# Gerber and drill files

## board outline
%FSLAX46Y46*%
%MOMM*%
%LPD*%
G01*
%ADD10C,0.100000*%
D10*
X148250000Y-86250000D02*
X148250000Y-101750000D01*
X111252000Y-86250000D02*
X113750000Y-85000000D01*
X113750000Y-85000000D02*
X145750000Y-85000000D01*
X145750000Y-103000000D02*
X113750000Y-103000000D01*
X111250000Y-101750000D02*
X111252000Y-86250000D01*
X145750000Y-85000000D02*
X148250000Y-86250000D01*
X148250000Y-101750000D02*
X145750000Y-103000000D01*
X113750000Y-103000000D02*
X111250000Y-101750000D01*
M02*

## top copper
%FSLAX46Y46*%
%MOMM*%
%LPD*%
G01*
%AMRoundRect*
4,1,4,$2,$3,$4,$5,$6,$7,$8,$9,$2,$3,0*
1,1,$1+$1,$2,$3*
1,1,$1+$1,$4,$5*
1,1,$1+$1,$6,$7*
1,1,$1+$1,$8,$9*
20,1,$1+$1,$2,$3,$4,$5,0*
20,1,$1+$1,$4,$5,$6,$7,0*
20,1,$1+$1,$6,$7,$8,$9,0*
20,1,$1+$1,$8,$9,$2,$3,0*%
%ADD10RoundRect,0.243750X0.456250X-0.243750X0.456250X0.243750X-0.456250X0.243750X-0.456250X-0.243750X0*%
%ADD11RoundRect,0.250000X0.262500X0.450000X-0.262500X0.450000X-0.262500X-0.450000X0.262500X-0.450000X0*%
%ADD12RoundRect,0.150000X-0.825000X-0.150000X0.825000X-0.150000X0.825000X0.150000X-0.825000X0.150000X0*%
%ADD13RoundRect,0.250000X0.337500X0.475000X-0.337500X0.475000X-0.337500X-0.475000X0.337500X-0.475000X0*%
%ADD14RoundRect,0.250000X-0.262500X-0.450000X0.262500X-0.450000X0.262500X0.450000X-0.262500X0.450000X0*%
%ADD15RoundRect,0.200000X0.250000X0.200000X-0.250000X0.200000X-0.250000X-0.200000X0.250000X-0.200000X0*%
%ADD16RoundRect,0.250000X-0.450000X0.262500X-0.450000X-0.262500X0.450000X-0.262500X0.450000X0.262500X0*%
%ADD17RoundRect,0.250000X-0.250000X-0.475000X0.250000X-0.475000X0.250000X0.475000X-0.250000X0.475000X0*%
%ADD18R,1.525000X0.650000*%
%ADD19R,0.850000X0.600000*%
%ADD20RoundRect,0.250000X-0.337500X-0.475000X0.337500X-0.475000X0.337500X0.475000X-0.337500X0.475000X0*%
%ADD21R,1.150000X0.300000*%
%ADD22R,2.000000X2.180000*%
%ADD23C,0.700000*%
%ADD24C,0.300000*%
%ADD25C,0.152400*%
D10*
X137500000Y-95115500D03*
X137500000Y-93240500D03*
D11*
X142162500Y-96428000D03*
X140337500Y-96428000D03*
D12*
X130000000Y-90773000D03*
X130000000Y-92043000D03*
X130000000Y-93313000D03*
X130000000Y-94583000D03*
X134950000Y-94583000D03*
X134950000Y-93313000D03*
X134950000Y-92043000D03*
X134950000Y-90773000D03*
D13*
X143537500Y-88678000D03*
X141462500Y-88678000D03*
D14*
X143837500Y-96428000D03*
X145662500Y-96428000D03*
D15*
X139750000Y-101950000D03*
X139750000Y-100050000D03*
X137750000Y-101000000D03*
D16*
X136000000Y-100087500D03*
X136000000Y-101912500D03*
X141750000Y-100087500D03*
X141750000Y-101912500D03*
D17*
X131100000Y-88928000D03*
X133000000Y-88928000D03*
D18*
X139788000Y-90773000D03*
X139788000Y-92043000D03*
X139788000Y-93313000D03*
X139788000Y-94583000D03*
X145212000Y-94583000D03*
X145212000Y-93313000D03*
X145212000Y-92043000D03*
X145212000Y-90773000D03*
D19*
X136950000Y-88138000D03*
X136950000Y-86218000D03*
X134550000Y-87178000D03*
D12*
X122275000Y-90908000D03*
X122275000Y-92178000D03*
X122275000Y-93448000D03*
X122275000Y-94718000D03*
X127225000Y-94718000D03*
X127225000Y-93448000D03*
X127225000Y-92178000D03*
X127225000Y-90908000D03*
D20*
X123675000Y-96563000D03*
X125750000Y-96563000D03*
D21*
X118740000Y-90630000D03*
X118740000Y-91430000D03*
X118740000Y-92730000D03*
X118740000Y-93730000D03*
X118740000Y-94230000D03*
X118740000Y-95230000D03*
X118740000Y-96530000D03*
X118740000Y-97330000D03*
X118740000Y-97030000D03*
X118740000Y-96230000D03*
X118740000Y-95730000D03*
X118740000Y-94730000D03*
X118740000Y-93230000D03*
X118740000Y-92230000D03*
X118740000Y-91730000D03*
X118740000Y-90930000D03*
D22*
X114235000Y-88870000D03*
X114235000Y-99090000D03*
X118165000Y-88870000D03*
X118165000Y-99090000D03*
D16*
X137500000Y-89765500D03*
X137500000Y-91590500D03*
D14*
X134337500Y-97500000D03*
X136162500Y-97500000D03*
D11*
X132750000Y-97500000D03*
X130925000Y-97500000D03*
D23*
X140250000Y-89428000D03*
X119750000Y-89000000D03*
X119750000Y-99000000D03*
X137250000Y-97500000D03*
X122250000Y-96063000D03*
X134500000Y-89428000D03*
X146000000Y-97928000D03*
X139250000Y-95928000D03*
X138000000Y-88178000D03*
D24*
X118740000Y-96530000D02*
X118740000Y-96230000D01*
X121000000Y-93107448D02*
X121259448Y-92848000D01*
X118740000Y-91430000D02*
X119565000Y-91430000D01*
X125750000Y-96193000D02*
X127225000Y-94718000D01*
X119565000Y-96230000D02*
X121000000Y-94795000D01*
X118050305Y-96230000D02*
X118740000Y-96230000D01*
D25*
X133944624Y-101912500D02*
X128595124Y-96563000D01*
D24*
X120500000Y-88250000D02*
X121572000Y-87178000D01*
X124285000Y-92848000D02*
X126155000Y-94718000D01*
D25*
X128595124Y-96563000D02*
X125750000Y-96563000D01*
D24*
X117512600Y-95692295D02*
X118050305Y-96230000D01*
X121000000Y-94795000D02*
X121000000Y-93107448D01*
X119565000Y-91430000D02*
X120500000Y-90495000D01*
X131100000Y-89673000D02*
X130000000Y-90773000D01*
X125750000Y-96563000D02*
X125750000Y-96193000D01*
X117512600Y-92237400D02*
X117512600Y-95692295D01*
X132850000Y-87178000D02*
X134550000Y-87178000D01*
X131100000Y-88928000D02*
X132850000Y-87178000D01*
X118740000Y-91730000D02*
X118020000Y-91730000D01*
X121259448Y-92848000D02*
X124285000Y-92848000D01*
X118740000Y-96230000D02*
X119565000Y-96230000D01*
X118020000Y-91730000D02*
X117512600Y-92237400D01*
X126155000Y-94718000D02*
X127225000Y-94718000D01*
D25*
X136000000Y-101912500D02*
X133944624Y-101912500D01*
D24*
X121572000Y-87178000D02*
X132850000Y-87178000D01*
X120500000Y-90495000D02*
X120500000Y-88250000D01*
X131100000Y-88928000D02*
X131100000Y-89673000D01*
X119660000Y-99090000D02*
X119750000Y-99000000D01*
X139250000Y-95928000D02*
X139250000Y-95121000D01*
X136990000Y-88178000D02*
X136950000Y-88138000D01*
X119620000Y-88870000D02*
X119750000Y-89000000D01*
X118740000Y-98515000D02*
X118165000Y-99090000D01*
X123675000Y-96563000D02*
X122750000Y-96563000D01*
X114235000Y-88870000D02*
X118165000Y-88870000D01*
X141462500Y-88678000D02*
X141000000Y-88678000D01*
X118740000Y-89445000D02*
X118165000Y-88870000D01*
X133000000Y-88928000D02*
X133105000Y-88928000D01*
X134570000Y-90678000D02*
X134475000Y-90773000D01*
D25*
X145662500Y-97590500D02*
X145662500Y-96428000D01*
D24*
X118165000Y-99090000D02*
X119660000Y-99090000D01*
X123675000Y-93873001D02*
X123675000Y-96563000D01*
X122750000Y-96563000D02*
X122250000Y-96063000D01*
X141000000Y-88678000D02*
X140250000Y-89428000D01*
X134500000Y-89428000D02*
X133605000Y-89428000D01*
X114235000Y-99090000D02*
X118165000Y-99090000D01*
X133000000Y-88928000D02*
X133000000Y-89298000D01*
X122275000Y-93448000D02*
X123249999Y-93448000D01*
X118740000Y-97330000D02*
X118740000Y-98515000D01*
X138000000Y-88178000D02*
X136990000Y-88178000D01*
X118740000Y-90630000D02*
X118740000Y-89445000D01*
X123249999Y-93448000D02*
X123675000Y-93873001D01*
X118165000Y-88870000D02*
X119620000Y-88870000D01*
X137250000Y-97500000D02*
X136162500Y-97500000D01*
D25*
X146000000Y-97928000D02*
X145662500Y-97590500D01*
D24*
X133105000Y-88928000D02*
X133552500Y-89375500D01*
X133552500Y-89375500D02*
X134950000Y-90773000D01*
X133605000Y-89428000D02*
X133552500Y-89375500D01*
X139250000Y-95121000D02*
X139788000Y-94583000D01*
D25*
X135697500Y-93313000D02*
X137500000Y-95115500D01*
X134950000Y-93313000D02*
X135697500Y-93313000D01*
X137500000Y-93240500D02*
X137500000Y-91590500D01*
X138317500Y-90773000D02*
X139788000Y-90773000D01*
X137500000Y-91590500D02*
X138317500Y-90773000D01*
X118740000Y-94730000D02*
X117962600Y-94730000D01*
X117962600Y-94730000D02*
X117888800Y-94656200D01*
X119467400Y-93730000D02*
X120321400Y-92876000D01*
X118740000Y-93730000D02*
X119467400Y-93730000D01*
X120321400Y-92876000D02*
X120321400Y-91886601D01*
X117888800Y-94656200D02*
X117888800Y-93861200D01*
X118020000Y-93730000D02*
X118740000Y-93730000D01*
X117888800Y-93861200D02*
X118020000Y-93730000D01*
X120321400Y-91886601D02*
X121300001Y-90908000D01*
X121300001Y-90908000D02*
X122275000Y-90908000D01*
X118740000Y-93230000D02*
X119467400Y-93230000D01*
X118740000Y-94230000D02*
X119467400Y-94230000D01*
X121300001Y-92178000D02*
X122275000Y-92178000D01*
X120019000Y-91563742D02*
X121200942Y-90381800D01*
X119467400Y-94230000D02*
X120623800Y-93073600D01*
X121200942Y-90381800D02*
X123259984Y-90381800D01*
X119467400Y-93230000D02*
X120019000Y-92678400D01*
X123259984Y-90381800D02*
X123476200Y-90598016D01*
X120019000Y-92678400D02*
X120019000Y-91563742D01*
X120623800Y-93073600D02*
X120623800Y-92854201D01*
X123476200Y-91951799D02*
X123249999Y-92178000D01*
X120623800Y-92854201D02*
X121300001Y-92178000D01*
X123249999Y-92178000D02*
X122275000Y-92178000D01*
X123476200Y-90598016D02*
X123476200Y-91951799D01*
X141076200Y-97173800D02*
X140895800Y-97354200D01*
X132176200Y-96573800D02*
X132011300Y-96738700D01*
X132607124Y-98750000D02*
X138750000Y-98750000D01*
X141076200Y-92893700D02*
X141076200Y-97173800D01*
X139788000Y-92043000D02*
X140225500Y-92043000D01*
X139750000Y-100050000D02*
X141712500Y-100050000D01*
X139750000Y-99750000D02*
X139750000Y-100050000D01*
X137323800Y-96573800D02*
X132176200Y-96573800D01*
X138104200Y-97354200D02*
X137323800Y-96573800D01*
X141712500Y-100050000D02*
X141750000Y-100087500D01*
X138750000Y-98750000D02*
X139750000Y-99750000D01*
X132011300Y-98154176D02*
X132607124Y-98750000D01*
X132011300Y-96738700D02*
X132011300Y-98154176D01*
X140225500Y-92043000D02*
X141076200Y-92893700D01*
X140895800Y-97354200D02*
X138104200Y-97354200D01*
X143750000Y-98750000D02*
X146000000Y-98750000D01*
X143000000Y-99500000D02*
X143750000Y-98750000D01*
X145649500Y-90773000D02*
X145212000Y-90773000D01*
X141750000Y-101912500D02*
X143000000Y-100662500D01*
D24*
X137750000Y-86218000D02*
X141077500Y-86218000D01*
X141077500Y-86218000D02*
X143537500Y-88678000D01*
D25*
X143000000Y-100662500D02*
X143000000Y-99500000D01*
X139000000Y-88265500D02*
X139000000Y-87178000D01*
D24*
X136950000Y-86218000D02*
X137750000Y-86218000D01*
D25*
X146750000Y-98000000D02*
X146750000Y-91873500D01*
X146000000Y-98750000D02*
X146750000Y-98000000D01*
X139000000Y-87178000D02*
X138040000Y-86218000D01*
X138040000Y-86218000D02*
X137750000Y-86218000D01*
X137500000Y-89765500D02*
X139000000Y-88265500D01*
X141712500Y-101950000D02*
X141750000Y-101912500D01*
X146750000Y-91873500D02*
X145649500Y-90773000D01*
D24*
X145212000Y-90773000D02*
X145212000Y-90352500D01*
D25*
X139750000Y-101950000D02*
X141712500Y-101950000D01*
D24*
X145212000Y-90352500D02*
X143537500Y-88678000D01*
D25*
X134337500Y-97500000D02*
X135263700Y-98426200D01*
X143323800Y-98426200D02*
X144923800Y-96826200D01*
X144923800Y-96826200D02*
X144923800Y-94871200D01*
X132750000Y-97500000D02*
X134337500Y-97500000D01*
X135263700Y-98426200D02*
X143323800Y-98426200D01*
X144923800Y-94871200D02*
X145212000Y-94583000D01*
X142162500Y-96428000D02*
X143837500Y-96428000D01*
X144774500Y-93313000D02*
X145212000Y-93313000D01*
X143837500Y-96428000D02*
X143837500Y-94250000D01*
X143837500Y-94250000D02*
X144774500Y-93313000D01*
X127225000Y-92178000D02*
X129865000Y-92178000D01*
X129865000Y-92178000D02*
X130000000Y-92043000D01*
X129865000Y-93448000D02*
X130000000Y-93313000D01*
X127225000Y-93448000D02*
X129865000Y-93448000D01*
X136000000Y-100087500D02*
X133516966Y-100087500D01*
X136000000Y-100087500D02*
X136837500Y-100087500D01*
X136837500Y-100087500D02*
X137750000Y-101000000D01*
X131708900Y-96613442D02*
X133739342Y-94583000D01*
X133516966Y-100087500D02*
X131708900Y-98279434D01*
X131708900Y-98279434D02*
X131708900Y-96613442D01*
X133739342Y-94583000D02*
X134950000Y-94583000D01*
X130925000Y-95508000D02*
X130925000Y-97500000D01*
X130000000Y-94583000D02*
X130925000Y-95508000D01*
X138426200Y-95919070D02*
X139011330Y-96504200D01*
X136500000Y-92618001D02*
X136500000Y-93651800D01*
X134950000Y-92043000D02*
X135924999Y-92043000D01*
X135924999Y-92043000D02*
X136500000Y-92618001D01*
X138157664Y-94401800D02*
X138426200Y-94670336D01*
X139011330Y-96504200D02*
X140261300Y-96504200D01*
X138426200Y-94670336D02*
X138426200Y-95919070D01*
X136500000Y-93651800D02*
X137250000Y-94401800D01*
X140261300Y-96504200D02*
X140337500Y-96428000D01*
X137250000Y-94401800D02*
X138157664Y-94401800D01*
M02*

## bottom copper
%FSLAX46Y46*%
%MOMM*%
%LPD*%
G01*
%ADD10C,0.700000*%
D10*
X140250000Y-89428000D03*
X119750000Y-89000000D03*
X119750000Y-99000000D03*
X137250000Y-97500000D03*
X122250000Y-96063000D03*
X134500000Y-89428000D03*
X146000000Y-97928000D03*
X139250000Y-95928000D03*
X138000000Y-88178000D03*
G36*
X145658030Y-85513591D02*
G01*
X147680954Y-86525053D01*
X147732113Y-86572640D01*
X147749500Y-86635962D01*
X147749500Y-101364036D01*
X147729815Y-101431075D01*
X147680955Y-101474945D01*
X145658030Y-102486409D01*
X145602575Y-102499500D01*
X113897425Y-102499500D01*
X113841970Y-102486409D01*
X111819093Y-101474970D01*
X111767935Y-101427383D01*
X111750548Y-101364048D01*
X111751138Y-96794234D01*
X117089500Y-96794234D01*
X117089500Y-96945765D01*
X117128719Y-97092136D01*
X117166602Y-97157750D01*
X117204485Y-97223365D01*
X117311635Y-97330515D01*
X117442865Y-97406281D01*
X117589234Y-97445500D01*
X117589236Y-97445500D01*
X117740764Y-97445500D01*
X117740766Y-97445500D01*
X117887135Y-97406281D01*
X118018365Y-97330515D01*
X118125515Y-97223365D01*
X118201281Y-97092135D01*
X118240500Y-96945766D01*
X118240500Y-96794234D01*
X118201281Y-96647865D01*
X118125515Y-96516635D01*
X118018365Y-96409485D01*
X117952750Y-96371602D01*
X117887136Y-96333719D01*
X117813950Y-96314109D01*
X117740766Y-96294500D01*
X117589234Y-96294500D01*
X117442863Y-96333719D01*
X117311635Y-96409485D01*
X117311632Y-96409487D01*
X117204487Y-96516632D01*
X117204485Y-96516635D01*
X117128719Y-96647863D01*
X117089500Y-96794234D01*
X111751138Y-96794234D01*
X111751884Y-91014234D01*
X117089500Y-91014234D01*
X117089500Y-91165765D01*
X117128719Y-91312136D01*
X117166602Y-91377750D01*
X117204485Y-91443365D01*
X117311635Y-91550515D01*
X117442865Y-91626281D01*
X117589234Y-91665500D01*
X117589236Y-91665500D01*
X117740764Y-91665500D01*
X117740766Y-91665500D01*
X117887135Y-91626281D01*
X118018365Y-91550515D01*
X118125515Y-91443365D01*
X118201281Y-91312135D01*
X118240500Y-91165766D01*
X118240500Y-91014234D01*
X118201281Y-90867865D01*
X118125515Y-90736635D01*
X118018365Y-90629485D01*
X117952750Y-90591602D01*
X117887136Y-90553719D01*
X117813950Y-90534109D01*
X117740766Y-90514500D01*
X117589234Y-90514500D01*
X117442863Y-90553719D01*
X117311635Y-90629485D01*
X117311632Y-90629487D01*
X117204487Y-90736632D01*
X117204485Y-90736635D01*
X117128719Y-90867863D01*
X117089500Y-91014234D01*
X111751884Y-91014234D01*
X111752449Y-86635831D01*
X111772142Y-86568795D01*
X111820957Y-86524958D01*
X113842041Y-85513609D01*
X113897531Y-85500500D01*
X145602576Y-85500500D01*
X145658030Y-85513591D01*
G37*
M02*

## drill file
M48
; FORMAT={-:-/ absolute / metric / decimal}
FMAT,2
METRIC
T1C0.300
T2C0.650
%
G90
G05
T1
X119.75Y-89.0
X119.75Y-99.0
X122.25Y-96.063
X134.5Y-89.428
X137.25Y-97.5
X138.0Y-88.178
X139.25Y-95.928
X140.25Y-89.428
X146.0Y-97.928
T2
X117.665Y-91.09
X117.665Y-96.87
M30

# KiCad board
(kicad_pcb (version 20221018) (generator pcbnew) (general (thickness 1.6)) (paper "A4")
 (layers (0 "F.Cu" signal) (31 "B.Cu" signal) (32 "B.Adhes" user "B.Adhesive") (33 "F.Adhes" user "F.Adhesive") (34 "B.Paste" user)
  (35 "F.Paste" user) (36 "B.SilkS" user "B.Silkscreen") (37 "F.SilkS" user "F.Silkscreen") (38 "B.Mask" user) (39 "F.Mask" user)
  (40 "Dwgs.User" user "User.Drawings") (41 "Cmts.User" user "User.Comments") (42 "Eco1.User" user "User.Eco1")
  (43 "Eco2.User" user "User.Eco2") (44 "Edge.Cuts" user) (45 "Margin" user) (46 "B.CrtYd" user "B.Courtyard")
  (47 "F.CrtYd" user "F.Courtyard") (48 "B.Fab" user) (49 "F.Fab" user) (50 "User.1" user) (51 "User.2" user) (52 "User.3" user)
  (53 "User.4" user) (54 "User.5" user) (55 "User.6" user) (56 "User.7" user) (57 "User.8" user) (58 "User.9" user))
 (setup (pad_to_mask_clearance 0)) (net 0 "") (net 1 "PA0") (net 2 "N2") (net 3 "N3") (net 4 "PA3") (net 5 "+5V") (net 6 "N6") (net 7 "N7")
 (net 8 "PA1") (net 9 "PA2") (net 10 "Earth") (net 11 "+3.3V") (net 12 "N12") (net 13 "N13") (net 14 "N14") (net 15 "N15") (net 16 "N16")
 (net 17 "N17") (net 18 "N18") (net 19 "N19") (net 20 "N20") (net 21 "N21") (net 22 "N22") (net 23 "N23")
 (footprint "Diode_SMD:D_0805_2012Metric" (layer "F.Cu") (at 137.5 94.178 90)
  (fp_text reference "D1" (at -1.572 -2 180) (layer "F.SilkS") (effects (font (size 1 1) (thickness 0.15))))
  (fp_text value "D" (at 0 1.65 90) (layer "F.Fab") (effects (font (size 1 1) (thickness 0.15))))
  (pad "1" smd roundrect (at -0.9375 0 90) (size 0.975 1.4) (layers "F.Cu" "F.Paste" "F.Mask") (roundrect_rratio 0.25) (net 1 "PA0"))
  (pad "2" smd roundrect (at 0.9375 0 90) (size 0.975 1.4) (layers "F.Cu" "F.Paste" "F.Mask") (roundrect_rratio 0.25) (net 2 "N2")))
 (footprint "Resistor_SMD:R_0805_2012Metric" (layer "F.Cu") (at 141.25 96.428 180)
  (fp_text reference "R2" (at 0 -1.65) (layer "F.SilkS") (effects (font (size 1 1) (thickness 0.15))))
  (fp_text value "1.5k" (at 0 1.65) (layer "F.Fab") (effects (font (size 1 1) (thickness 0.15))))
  (pad "1" smd roundrect (at -0.9125 0 180) (size 1.025 1.4) (layers "F.Cu" "F.Paste" "F.Mask") (roundrect_rratio 0.243902) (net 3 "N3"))
  (pad "2" smd roundrect (at 0.9125 0 180) (size 1.025 1.4) (layers "F.Cu" "F.Paste" "F.Mask") (roundrect_rratio 0.243902) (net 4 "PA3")))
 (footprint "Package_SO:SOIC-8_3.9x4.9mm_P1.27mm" (layer "F.Cu") (at 132.475 92.678)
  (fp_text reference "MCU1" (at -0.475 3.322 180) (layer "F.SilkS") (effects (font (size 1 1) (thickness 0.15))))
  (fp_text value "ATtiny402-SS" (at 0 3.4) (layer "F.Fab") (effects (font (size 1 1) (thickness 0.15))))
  (pad "1" smd roundrect (at -2.475 -1.905) (size 1.95 0.6) (layers "F.Cu" "F.Paste" "F.Mask") (roundrect_rratio 0.25) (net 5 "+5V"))
  (pad "2" smd roundrect (at -2.475 -0.635) (size 1.95 0.6) (layers "F.Cu" "F.Paste" "F.Mask") (roundrect_rratio 0.25) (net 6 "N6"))
  (pad "3" smd roundrect (at -2.475 0.635) (size 1.95 0.6) (layers "F.Cu" "F.Paste" "F.Mask") (roundrect_rratio 0.25) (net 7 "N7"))
  (pad "4" smd roundrect (at -2.475 1.905) (size 1.95 0.6) (layers "F.Cu" "F.Paste" "F.Mask") (roundrect_rratio 0.25) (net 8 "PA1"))
  (pad "5" smd roundrect (at 2.475 1.905) (size 1.95 0.6) (layers "F.Cu" "F.Paste" "F.Mask") (roundrect_rratio 0.25) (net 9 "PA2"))
  (pad "6" smd roundrect (at 2.475 0.635) (size 1.95 0.6) (layers "F.Cu" "F.Paste" "F.Mask") (roundrect_rratio 0.25) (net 1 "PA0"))
  (pad "7" smd roundrect (at 2.475 -0.635) (size 1.95 0.6) (layers "F.Cu" "F.Paste" "F.Mask") (roundrect_rratio 0.25) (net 4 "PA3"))
  (pad "8" smd roundrect (at 2.475 -1.905) (size 1.95 0.6) (layers "F.Cu" "F.Paste" "F.Mask") (roundrect_rratio 0.25) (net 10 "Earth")))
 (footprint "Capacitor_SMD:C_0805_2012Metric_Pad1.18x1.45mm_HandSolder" (layer "F.Cu") (at 142.5 88.678 180)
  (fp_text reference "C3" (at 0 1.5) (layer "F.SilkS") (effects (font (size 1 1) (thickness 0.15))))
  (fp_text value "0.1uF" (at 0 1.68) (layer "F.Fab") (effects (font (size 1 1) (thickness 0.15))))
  (pad "1" smd roundrect (at -1.0375 0 180) (size 1.175 1.45) (layers "F.Cu" "F.Paste" "F.Mask") (roundrect_rratio 0.212766)
   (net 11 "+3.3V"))
  (pad "2" smd roundrect (at 1.0375 0 180) (size 1.175 1.45) (layers "F.Cu" "F.Paste" "F.Mask") (roundrect_rratio 0.212766) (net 10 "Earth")))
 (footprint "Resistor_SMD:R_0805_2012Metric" (layer "F.Cu") (at 144.75 96.428)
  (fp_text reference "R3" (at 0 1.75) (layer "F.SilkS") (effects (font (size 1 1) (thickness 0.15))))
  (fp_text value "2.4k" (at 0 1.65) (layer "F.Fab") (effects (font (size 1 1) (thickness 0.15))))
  (pad "1" smd roundrect (at -0.9125 0) (size 1.025 1.4) (layers "F.Cu" "F.Paste" "F.Mask") (roundrect_rratio 0.243902) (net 3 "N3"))
  (pad "2" smd roundrect (at 0.9125 0) (size 1.025 1.4) (layers "F.Cu" "F.Paste" "F.Mask") (roundrect_rratio 0.243902) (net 10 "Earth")))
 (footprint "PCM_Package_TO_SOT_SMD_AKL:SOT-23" (layer "F.Cu") (at 138.75 101 180)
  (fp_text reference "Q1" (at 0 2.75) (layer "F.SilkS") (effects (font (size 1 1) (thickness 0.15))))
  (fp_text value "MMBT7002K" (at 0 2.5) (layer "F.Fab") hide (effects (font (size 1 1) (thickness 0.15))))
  (pad "1" smd roundrect (at -1 -0.95 180) (size 0.9 0.8) (layers "F.Cu" "F.Paste" "F.Mask") (roundrect_rratio 0.25) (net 11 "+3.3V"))
  (pad "2" smd roundrect (at -1 0.95 180) (size 0.9 0.8) (layers "F.Cu" "F.Paste" "F.Mask") (roundrect_rratio 0.25) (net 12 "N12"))
  (pad "3" smd roundrect (at 1 0 180) (size 0.9 0.8) (layers "F.Cu" "F.Paste" "F.Mask") (roundrect_rratio 0.25) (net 9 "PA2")))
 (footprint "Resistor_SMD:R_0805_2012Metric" (layer "F.Cu") (at 136 101 -90)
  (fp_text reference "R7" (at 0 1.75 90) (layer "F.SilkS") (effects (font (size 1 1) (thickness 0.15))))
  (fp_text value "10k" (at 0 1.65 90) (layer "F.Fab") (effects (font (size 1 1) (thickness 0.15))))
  (pad "1" smd roundrect (at -0.9125 0 270) (size 1.025 1.4) (layers "F.Cu" "F.Paste" "F.Mask") (roundrect_rratio 0.243902) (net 9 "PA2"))
  (pad "2" smd roundrect (at 0.9125 0 270) (size 1.025 1.4) (layers "F.Cu" "F.Paste" "F.Mask") (roundrect_rratio 0.243902) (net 5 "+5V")))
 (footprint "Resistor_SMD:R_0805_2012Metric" (layer "F.Cu") (at 141.75 101 -90)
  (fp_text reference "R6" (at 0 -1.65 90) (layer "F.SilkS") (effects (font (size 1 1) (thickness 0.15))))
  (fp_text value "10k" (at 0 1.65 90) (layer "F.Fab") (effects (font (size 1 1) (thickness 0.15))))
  (pad "1" smd roundrect (at -0.9125 0 270) (size 1.025 1.4) (layers "F.Cu" "F.Paste" "F.Mask") (roundrect_rratio 0.243902) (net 12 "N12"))
  (pad "2" smd roundrect (at 0.9125 0 270) (size 1.025 1.4) (layers "F.Cu" "F.Paste" "F.Mask") (roundrect_rratio 0.243902) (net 11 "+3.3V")))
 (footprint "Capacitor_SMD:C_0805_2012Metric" (layer "F.Cu") (at 132.05 88.928)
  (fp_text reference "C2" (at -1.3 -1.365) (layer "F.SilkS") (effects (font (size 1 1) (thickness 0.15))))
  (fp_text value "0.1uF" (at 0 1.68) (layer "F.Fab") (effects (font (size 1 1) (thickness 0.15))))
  (pad "1" smd roundrect (at -0.95 0) (size 1 1.45) (layers "F.Cu" "F.Paste" "F.Mask") (roundrect_rratio 0.25) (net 5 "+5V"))
  (pad "2" smd roundrect (at 0.95 0) (size 1 1.45) (layers "F.Cu" "F.Paste" "F.Mask") (roundrect_rratio 0.25) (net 10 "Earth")))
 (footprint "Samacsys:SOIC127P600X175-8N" (layer "F.Cu") (at 142.5 92.678)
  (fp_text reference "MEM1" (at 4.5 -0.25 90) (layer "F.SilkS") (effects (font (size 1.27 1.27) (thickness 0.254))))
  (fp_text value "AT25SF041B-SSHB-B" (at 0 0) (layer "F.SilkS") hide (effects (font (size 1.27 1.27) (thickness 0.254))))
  (pad "1" smd rect (at -2.712 -1.905 90) (size 0.65 1.525) (layers "F.Cu" "F.Paste" "F.Mask") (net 2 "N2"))
  (pad "2" smd rect (at -2.712 -0.635 90) (size 0.65 1.525) (layers "F.Cu" "F.Paste" "F.Mask") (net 12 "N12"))
  (pad "3" smd rect (at -2.712 0.635 90) (size 0.65 1.525) (layers "F.Cu" "F.Paste" "F.Mask") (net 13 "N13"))
  (pad "4" smd rect (at -2.712 1.905 90) (size 0.65 1.525) (layers "F.Cu" "F.Paste" "F.Mask") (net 10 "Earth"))
  (pad "5" smd rect (at 2.712 1.905 90) (size 0.65 1.525) (layers "F.Cu" "F.Paste" "F.Mask") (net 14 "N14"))
  (pad "6" smd rect (at 2.712 0.635 90) (size 0.65 1.525) (layers "F.Cu" "F.Paste" "F.Mask") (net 3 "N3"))
  (pad "7" smd rect (at 2.712 -0.635 90) (size 0.65 1.525) (layers "F.Cu" "F.Paste" "F.Mask") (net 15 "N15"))
  (pad "8" smd rect (at 2.712 -1.905 90) (size 0.65 1.525) (layers "F.Cu" "F.Paste" "F.Mask") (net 11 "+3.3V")))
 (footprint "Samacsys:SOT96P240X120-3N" (layer "F.Cu") (at 135.75 87.178 180)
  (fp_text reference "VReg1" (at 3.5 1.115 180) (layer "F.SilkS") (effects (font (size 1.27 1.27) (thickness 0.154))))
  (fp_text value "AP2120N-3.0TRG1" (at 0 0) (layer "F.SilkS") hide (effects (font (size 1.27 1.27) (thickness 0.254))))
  (pad "1" smd rect (at -1.2 -0.96 270) (size 0.6 0.85) (layers "F.Cu" "F.Paste" "F.Mask") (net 10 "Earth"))
  (pad "2" smd rect (at -1.2 0.96 270) (size 0.6 0.85) (layers "F.Cu" "F.Paste" "F.Mask") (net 11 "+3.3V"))
  (pad "3" smd rect (at 1.2 0 270) (size 0.6 0.85) (layers "F.Cu" "F.Paste" "F.Mask") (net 5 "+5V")))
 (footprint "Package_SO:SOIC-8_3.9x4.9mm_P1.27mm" (layer "F.Cu") (at 124.75 92.813)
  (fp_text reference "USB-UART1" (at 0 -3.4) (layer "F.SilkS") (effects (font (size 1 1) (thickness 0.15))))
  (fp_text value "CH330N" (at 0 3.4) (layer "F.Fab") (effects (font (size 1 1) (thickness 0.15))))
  (pad "1" smd roundrect (at -2.475 -1.905) (size 1.95 0.6) (layers "F.Cu" "F.Paste" "F.Mask") (roundrect_rratio 0.25) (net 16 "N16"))
  (pad "2" smd roundrect (at -2.475 -0.635) (size 1.95 0.6) (layers "F.Cu" "F.Paste" "F.Mask") (roundrect_rratio 0.25) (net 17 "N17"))
  (pad "3" smd roundrect (at -2.475 0.635) (size 1.95 0.6) (layers "F.Cu" "F.Paste" "F.Mask") (roundrect_rratio 0.25) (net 10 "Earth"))
  (pad "4" smd roundrect (at -2.475 1.905) (size 1.95 0.6) (layers "F.Cu" "F.Paste" "F.Mask") (roundrect_rratio 0.25) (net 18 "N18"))
  (pad "5" smd roundrect (at 2.475 1.905) (size 1.95 0.6) (layers "F.Cu" "F.Paste" "F.Mask") (roundrect_rratio 0.25) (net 5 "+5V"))
  (pad "6" smd roundrect (at 2.475 0.635) (size 1.95 0.6) (layers "F.Cu" "F.Paste" "F.Mask") (roundrect_rratio 0.25) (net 7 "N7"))
  (pad "7" smd roundrect (at 2.475 -0.635) (size 1.95 0.6) (layers "F.Cu" "F.Paste" "F.Mask") (roundrect_rratio 0.25) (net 6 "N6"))
  (pad "8" smd roundrect (at 2.475 -1.905) (size 1.95 0.6) (layers "F.Cu" "F.Paste" "F.Mask") (roundrect_rratio 0.25) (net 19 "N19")))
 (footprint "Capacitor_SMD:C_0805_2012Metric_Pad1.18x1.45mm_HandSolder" (layer "F.Cu") (at 124.7125 96.563)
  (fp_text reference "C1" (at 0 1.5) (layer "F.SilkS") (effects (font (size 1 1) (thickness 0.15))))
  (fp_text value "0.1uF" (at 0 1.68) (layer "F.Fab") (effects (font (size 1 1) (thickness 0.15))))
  (pad "1" smd roundrect (at -1.0375 0) (size 1.175 1.45) (layers "F.Cu" "F.Paste" "F.Mask") (roundrect_rratio 0.212766) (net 10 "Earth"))
  (pad "2" smd roundrect (at 1.0375 0) (size 1.175 1.45) (layers "F.Cu" "F.Paste" "F.Mask") (roundrect_rratio 0.212766) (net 5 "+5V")))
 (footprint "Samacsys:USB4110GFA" (layer "F.Cu") (at 115.062 93.98 -90)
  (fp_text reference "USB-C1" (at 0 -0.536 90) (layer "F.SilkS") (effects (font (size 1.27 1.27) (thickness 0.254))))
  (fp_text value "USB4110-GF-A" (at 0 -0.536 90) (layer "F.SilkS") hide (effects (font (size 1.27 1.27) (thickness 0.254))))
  (pad "" np_thru_hole circle (at -2.89 -2.603 270) (size 0.65 0.65) (drill 0.65) (layers "*.Cu" "*.Mask"))
  (pad "" np_thru_hole circle (at 2.89 -2.603 270) (size 0.65 0.65) (drill 0.65) (layers "*.Cu" "*.Mask"))
  (pad "A1" smd rect (at -3.35 -3.678 270) (size 0.3 1.15) (layers "F.Cu" "F.Paste" "F.Mask") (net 10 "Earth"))
  (pad "A4" smd rect (at -2.55 -3.678 270) (size 0.3 1.15) (layers "F.Cu" "F.Paste" "F.Mask") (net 5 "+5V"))
  (pad "A5" smd rect (at -1.25 -3.678 270) (size 0.3 1.15) (layers "F.Cu" "F.Paste" "F.Mask") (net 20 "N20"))
  (pad "A6" smd rect (at -0.25 -3.678 270) (size 0.3 1.15) (layers "F.Cu" "F.Paste" "F.Mask") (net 16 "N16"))
  (pad "A7" smd rect (at 0.25 -3.678 270) (size 0.3 1.15) (layers "F.Cu" "F.Paste" "F.Mask") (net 17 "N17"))
  (pad "A8" smd rect (at 1.25 -3.678 270) (size 0.3 1.15) (layers "F.Cu" "F.Paste" "F.Mask") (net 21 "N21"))
  (pad "A9" smd rect (at 2.55 -3.678 270) (size 0.3 1.15) (layers "F.Cu" "F.Paste" "F.Mask") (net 5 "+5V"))
  (pad "A12" smd rect (at 3.35 -3.678 270) (size 0.3 1.15) (layers "F.Cu" "F.Paste" "F.Mask") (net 10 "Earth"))
  (pad "B1" smd rect (at 3.05 -3.678 270) (size 0.3 1.15) (layers "F.Cu" "F.Paste" "F.Mask") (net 10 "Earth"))
  (pad "B4" smd rect (at 2.25 -3.678 270) (size 0.3 1.15) (layers "F.Cu" "F.Paste" "F.Mask") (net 5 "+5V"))
  (pad "B5" smd rect (at 1.75 -3.678 270) (size 0.3 1.15) (layers "F.Cu" "F.Paste" "F.Mask") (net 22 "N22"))
  (pad "B6" smd rect (at 0.75 -3.678 270) (size 0.3 1.15) (layers "F.Cu" "F.Paste" "F.Mask") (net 16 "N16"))
  (pad "B7" smd rect (at -0.75 -3.678 270) (size 0.3 1.15) (layers "F.Cu" "F.Paste" "F.Mask") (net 17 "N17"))
  (pad "B8" smd rect (at -1.75 -3.678 270) (size 0.3 1.15) (layers "F.Cu" "F.Paste" "F.Mask") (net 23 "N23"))
  (pad "B9" smd rect (at -2.25 -3.678 270) (size 0.3 1.15) (layers "F.Cu" "F.Paste" "F.Mask") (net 5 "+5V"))
  (pad "B12" smd rect (at -3.05 -3.678 270) (size 0.3 1.15) (layers "F.Cu" "F.Paste" "F.Mask") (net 10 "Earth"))
  (pad "MP1" smd rect (at -5.11 0.827) (size 2 2.18) (layers "F.Cu" "F.Paste" "F.Mask") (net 10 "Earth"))
  (pad "MP2" smd rect (at 5.11 0.827) (size 2 2.18) (layers "F.Cu" "F.Paste" "F.Mask") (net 10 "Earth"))
  (pad "MP3" smd rect (at -5.11 -3.103) (size 2 2.18) (layers "F.Cu" "F.Paste" "F.Mask") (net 10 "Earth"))
  (pad "MP4" smd rect (at 5.11 -3.103) (size 2 2.18) (layers "F.Cu" "F.Paste" "F.Mask") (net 10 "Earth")))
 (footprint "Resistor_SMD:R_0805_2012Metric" (layer "F.Cu") (at 137.5 90.678 -90)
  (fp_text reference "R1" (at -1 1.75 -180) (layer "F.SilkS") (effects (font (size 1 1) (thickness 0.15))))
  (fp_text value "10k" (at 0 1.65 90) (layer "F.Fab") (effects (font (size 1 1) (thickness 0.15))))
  (pad "1" smd roundrect (at -0.9125 0 270) (size 1.025 1.4) (layers "F.Cu" "F.Paste" "F.Mask") (roundrect_rratio 0.243902) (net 11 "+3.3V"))
  (pad "2" smd roundrect (at 0.9125 0 270) (size 1.025 1.4) (layers "F.Cu" "F.Paste" "F.Mask") (roundrect_rratio 0.243902) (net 2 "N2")))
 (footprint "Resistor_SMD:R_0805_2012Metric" (layer "F.Cu") (at 135.25 97.5)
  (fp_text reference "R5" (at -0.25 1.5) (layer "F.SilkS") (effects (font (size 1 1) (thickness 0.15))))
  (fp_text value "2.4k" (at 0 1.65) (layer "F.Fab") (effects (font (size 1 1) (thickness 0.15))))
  (pad "1" smd roundrect (at -0.9125 0) (size 1.025 1.4) (layers "F.Cu" "F.Paste" "F.Mask") (roundrect_rratio 0.243902) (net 14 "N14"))
  (pad "2" smd roundrect (at 0.9125 0) (size 1.025 1.4) (layers "F.Cu" "F.Paste" "F.Mask") (roundrect_rratio 0.243902) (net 10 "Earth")))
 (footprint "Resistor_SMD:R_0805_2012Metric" (layer "F.Cu") (at 131.8375 97.5 180)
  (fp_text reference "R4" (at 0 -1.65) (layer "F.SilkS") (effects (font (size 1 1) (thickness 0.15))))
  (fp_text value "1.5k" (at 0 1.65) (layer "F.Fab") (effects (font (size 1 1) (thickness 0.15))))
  (pad "1" smd roundrect (at -0.9125 0 180) (size 1.025 1.4) (layers "F.Cu" "F.Paste" "F.Mask") (roundrect_rratio 0.243902) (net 14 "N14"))
  (pad "2" smd roundrect (at 0.9125 0 180) (size 1.025 1.4) (layers "F.Cu" "F.Paste" "F.Mask") (roundrect_rratio 0.243902) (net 8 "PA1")))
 (gr_line (start 148.25 86.25) (end 148.25 101.75) (stroke (width 0.1) (type default)) (layer "Edge.Cuts"))
 (gr_line (start 111.252 86.25) (end 113.75 85) (stroke (width 0.1) (type default)) (layer "Edge.Cuts"))
 (gr_line (start 113.75 85) (end 145.75 85) (stroke (width 0.1) (type default)) (layer "Edge.Cuts"))
 (gr_line (start 145.75 103) (end 113.75 103) (stroke (width 0.1) (type default)) (layer "Edge.Cuts"))
 (gr_line (start 111.25 101.75) (end 111.252 86.25) (stroke (width 0.1) (type default)) (layer "Edge.Cuts"))
 (gr_line (start 145.75 85) (end 148.25 86.25) (stroke (width 0.1) (type default)) (layer "Edge.Cuts"))
 (gr_line (start 148.25 101.75) (end 145.75 103) (stroke (width 0.1) (type default)) (layer "Edge.Cuts"))
 (gr_line (start 113.75 103) (end 111.25 101.75) (stroke (width 0.1) (type default)) (layer "Edge.Cuts"))
 (segment (start 118.74 96.53) (end 118.74 96.23) (width 0.3) (layer "F.Cu") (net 5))
 (segment (start 121 93.107448) (end 121.259448 92.848) (width 0.3) (layer "F.Cu") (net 5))
 (segment (start 118.74 91.43) (end 119.565 91.43) (width 0.3) (layer "F.Cu") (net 5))
 (segment (start 125.75 96.193) (end 127.225 94.718) (width 0.3) (layer "F.Cu") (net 5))
 (segment (start 119.565 96.23) (end 121 94.795) (width 0.3) (layer "F.Cu") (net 5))
 (segment (start 118.050305 96.23) (end 118.74 96.23) (width 0.3) (layer "F.Cu") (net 5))
 (segment (start 133.944624 101.9125) (end 128.595124 96.563) (width 0.1524) (layer "F.Cu") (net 5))
 (segment (start 120.5 88.25) (end 121.572 87.178) (width 0.3) (layer "F.Cu") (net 5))
 (segment (start 124.285 92.848) (end 126.155 94.718) (width 0.3) (layer "F.Cu") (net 5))
 (segment (start 128.595124 96.563) (end 125.75 96.563) (width 0.1524) (layer "F.Cu") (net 5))
 (segment (start 117.5126 95.692295) (end 118.050305 96.23) (width 0.3) (layer "F.Cu") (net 5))
 (segment (start 121 94.795) (end 121 93.107448) (width 0.3) (layer "F.Cu") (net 5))
 (segment (start 119.565 91.43) (end 120.5 90.495) (width 0.3) (layer "F.Cu") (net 5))
 (segment (start 131.1 89.673) (end 130 90.773) (width 0.3) (layer "F.Cu") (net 5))
 (segment (start 125.75 96.563) (end 125.75 96.193) (width 0.3) (layer "F.Cu") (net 5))
 (segment (start 117.5126 92.2374) (end 117.5126 95.692295) (width 0.3) (layer "F.Cu") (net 5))
 (segment (start 132.85 87.178) (end 134.55 87.178) (width 0.3) (layer "F.Cu") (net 5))
 (segment (start 131.1 88.928) (end 132.85 87.178) (width 0.3) (layer "F.Cu") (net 5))
 (segment (start 118.74 91.73) (end 118.02 91.73) (width 0.3) (layer "F.Cu") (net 5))
 (segment (start 121.259448 92.848) (end 124.285 92.848) (width 0.3) (layer "F.Cu") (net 5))
 (segment (start 118.74 96.23) (end 119.565 96.23) (width 0.3) (layer "F.Cu") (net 5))
 (segment (start 118.02 91.73) (end 117.5126 92.2374) (width 0.3) (layer "F.Cu") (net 5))
 (segment (start 126.155 94.718) (end 127.225 94.718) (width 0.3) (layer "F.Cu") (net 5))
 (segment (start 136 101.9125) (end 133.944624 101.9125) (width 0.1524) (layer "F.Cu") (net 5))
 (segment (start 121.572 87.178) (end 132.85 87.178) (width 0.3) (layer "F.Cu") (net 5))
 (segment (start 120.5 90.495) (end 120.5 88.25) (width 0.3) (layer "F.Cu") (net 5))
 (segment (start 131.1 88.928) (end 131.1 89.673) (width 0.3) (layer "F.Cu") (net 5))
 (segment (start 119.66 99.09) (end 119.75 99) (width 0.3) (layer "F.Cu") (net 10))
 (segment (start 139.25 95.928) (end 139.25 95.121) (width 0.3) (layer "F.Cu") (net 10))
 (segment (start 136.99 88.178) (end 136.95 88.138) (width 0.3) (layer "F.Cu") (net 10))
 (segment (start 119.62 88.87) (end 119.75 89) (width 0.3) (layer "F.Cu") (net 10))
 (segment (start 118.74 98.515) (end 118.165 99.09) (width 0.3) (layer "F.Cu") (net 10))
 (segment (start 123.675 96.563) (end 122.75 96.563) (width 0.3) (layer "F.Cu") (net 10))
 (segment (start 114.235 88.87) (end 118.165 88.87) (width 0.3) (layer "F.Cu") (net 10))
 (segment (start 141.4625 88.678) (end 141 88.678) (width 0.3) (layer "F.Cu") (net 10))
 (segment (start 118.74 89.445) (end 118.165 88.87) (width 0.3) (layer "F.Cu") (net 10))
 (segment (start 133 88.928) (end 133.105 88.928) (width 0.3) (layer "F.Cu") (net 10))
 (segment (start 134.57 90.678) (end 134.475 90.773) (width 0.3) (layer "F.Cu") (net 10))
 (segment (start 145.6625 97.5905) (end 145.6625 96.428) (width 0.1524) (layer "F.Cu") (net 10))
 (segment (start 118.165 99.09) (end 119.66 99.09) (width 0.3) (layer "F.Cu") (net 10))
 (segment (start 123.675 93.873001) (end 123.675 96.563) (width 0.3) (layer "F.Cu") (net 10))
 (segment (start 122.75 96.563) (end 122.25 96.063) (width 0.3) (layer "F.Cu") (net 10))
 (segment (start 141 88.678) (end 140.25 89.428) (width 0.3) (layer "F.Cu") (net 10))
 (segment (start 134.5 89.428) (end 133.605 89.428) (width 0.3) (layer "F.Cu") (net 10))
 (segment (start 114.235 99.09) (end 118.165 99.09) (width 0.3) (layer "F.Cu") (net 10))
 (segment (start 133 88.928) (end 133 89.298) (width 0.3) (layer "F.Cu") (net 10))
 (segment (start 122.275 93.448) (end 123.249999 93.448) (width 0.3) (layer "F.Cu") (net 10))
 (segment (start 118.74 97.33) (end 118.74 98.515) (width 0.3) (layer "F.Cu") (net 10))
 (segment (start 138 88.178) (end 136.99 88.178) (width 0.3) (layer "F.Cu") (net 10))
 (segment (start 118.74 90.63) (end 118.74 89.445) (width 0.3) (layer "F.Cu") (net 10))
 (segment (start 123.249999 93.448) (end 123.675 93.873001) (width 0.3) (layer "F.Cu") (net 10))
 (segment (start 118.165 88.87) (end 119.62 88.87) (width 0.3) (layer "F.Cu") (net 10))
 (segment (start 137.25 97.5) (end 136.1625 97.5) (width 0.3) (layer "F.Cu") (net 10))
 (segment (start 146 97.928) (end 145.6625 97.5905) (width 0.1524) (layer "F.Cu") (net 10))
 (segment (start 133.105 88.928) (end 133.5525 89.3755) (width 0.3) (layer "F.Cu") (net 10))
 (segment (start 133.5525 89.3755) (end 134.95 90.773) (width 0.3) (layer "F.Cu") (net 10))
 (segment (start 133.605 89.428) (end 133.5525 89.3755) (width 0.3) (layer "F.Cu") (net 10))
 (segment (start 139.25 95.121) (end 139.788 94.583) (width 0.3) (layer "F.Cu") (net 10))
 (via (at 140.25 89.428) (size 0.7) (drill 0.3) (layers "F.Cu" "B.Cu") (free) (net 10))
 (via (at 119.75 89) (size 0.7) (drill 0.3) (layers "F.Cu" "B.Cu") (free) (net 10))
 (via (at 119.75 99) (size 0.7) (drill 0.3) (layers "F.Cu" "B.Cu") (free) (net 10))
 (via (at 137.25 97.5) (size 0.7) (drill 0.3) (layers "F.Cu" "B.Cu") (free) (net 10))
 (via (at 122.25 96.063) (size 0.7) (drill 0.3) (layers "F.Cu" "B.Cu") (free) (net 10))
 (via (at 134.5 89.428) (size 0.7) (drill 0.3) (layers "F.Cu" "B.Cu") (free) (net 10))
 (via (at 146 97.928) (size 0.7) (drill 0.3) (layers "F.Cu" "B.Cu") (free) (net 10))
 (via (at 139.25 95.928) (size 0.7) (drill 0.3) (layers "F.Cu" "B.Cu") (free) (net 10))
 (via (at 138 88.178) (size 0.7) (drill 0.3) (layers "F.Cu" "B.Cu") (free) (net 10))
 (segment (start 135.6975 93.313) (end 137.5 95.1155) (width 0.1524) (layer "F.Cu") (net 1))
 (segment (start 134.95 93.313) (end 135.6975 93.313) (width 0.1524) (layer "F.Cu") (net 1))
 (segment (start 137.5 93.2405) (end 137.5 91.5905) (width 0.1524) (layer "F.Cu") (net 2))
 (segment (start 138.3175 90.773) (end 139.788 90.773) (width 0.1524) (layer "F.Cu") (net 2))
 (segment (start 137.5 91.5905) (end 138.3175 90.773) (width 0.1524) (layer "F.Cu") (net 2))
 (segment (start 118.74 94.73) (end 117.9626 94.73) (width 0.1524) (layer "F.Cu") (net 16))
 (segment (start 117.9626 94.73) (end 117.8888 94.6562) (width 0.1524) (layer "F.Cu") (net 16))
 (segment (start 119.4674 93.73) (end 120.3214 92.876) (width 0.1524) (layer "F.Cu") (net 16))
 (segment (start 118.74 93.73) (end 119.4674 93.73) (width 0.1524) (layer "F.Cu") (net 16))
 (segment (start 120.3214 92.876) (end 120.3214 91.886601) (width 0.1524) (layer "F.Cu") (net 16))
 (segment (start 117.8888 94.6562) (end 117.8888 93.8612) (width 0.1524) (layer "F.Cu") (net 16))
 (segment (start 118.02 93.73) (end 118.74 93.73) (width 0.1524) (layer "F.Cu") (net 16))
 (segment (start 117.8888 93.8612) (end 118.02 93.73) (width 0.1524) (layer "F.Cu") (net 16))
 (segment (start 120.3214 91.886601) (end 121.300001 90.908) (width 0.1524) (layer "F.Cu") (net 16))
 (segment (start 121.300001 90.908) (end 122.275 90.908) (width 0.1524) (layer "F.Cu") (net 16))
 (segment (start 118.74 93.23) (end 119.4674 93.23) (width 0.1524) (layer "F.Cu") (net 17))
 (segment (start 118.74 94.23) (end 119.4674 94.23) (width 0.1524) (layer "F.Cu") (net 17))
 (segment (start 121.300001 92.178) (end 122.275 92.178) (width 0.1524) (layer "F.Cu") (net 17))
 (segment (start 120.019 91.563742) (end 121.200942 90.3818) (width 0.1524) (layer "F.Cu") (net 17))
 (segment (start 119.4674 94.23) (end 120.6238 93.0736) (width 0.1524) (layer "F.Cu") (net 17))
 (segment (start 121.200942 90.3818) (end 123.259984 90.3818) (width 0.1524) (layer "F.Cu") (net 17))
 (segment (start 119.4674 93.23) (end 120.019 92.6784) (width 0.1524) (layer "F.Cu") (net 17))
 (segment (start 123.259984 90.3818) (end 123.4762 90.598016) (width 0.1524) (layer "F.Cu") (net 17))
 (segment (start 120.019 92.6784) (end 120.019 91.563742) (width 0.1524) (layer "F.Cu") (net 17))
 (segment (start 120.6238 93.0736) (end 120.6238 92.854201) (width 0.1524) (layer "F.Cu") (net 17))
 (segment (start 123.4762 91.951799) (end 123.249999 92.178) (width 0.1524) (layer "F.Cu") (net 17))
 (segment (start 120.6238 92.854201) (end 121.300001 92.178) (width 0.1524) (layer "F.Cu") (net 17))
 (segment (start 123.249999 92.178) (end 122.275 92.178) (width 0.1524) (layer "F.Cu") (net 17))
 (segment (start 123.4762 90.598016) (end 123.4762 91.951799) (width 0.1524) (layer "F.Cu") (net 17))
 (segment (start 141.0762 97.1738) (end 140.8958 97.3542) (width 0.1524) (layer "F.Cu") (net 12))
 (segment (start 132.1762 96.5738) (end 132.0113 96.7387) (width 0.1524) (layer "F.Cu") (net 12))
 (segment (start 132.607124 98.75) (end 138.75 98.75) (width 0.1524) (layer "F.Cu") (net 12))
 (segment (start 141.0762 92.8937) (end 141.0762 97.1738) (width 0.1524) (layer "F.Cu") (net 12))
 (segment (start 139.788 92.043) (end 140.2255 92.043) (width 0.1524) (layer "F.Cu") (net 12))
 (segment (start 139.75 100.05) (end 141.7125 100.05) (width 0.1524) (layer "F.Cu") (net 12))
 (segment (start 139.75 99.75) (end 139.75 100.05) (width 0.1524) (layer "F.Cu") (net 12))
 (segment (start 137.3238 96.5738) (end 132.1762 96.5738) (width 0.1524) (layer "F.Cu") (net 12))
 (segment (start 138.1042 97.3542) (end 137.3238 96.5738) (width 0.1524) (layer "F.Cu") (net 12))
 (segment (start 141.7125 100.05) (end 141.75 100.0875) (width 0.1524) (layer "F.Cu") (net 12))
 (segment (start 138.75 98.75) (end 139.75 99.75) (width 0.1524) (layer "F.Cu") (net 12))
 (segment (start 132.0113 98.154176) (end 132.607124 98.75) (width 0.1524) (layer "F.Cu") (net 12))
 (segment (start 132.0113 96.7387) (end 132.0113 98.154176) (width 0.1524) (layer "F.Cu") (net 12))
 (segment (start 140.2255 92.043) (end 141.0762 92.8937) (width 0.1524) (layer "F.Cu") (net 12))
 (segment (start 140.8958 97.3542) (end 138.1042 97.3542) (width 0.1524) (layer "F.Cu") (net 12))
 (segment (start 143.75 98.75) (end 146 98.75) (width 0.1524) (layer "F.Cu") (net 11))
 (segment (start 143 99.5) (end 143.75 98.75) (width 0.1524) (layer "F.Cu") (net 11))
 (segment (start 145.6495 90.773) (end 145.212 90.773) (width 0.1524) (layer "F.Cu") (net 11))
 (segment (start 141.75 101.9125) (end 143 100.6625) (width 0.1524) (layer "F.Cu") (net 11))
 (segment (start 137.75 86.218) (end 141.0775 86.218) (width 0.3) (layer "F.Cu") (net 11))
 (segment (start 141.0775 86.218) (end 143.5375 88.678) (width 0.3) (layer "F.Cu") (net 11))
 (segment (start 143 100.6625) (end 143 99.5) (width 0.1524) (layer "F.Cu") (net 11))
 (segment (start 139 88.2655) (end 139 87.178) (width 0.1524) (layer "F.Cu") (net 11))
 (segment (start 136.95 86.218) (end 137.75 86.218) (width 0.3) (layer "F.Cu") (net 11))
 (segment (start 146.75 98) (end 146.75 91.8735) (width 0.1524) (layer "F.Cu") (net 11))
 (segment (start 146 98.75) (end 146.75 98) (width 0.1524) (layer "F.Cu") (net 11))
 (segment (start 139 87.178) (end 138.04 86.218) (width 0.1524) (layer "F.Cu") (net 11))
 (segment (start 138.04 86.218) (end 137.75 86.218) (width 0.1524) (layer "F.Cu") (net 11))
 (segment (start 137.5 89.7655) (end 139 88.2655) (width 0.1524) (layer "F.Cu") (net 11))
 (segment (start 141.7125 101.95) (end 141.75 101.9125) (width 0.1524) (layer "F.Cu") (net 11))
 (segment (start 146.75 91.8735) (end 145.6495 90.773) (width 0.1524) (layer "F.Cu") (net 11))
 (segment (start 145.212 90.773) (end 145.212 90.3525) (width 0.3) (layer "F.Cu") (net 11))
 (segment (start 139.75 101.95) (end 141.7125 101.95) (width 0.1524) (layer "F.Cu") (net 11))
 (segment (start 145.212 90.3525) (end 143.5375 88.678) (width 0.3) (layer "F.Cu") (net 11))
 (segment (start 134.3375 97.5) (end 135.2637 98.4262) (width 0.1524) (layer "F.Cu") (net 14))
 (segment (start 143.3238 98.4262) (end 144.9238 96.8262) (width 0.1524) (layer "F.Cu") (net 14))
 (segment (start 144.9238 96.8262) (end 144.9238 94.8712) (width 0.1524) (layer "F.Cu") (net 14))
 (segment (start 132.75 97.5) (end 134.3375 97.5) (width 0.1524) (layer "F.Cu") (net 14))
 (segment (start 135.2637 98.4262) (end 143.3238 98.4262) (width 0.1524) (layer "F.Cu") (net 14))
 (segment (start 144.9238 94.8712) (end 145.212 94.583) (width 0.1524) (layer "F.Cu") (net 14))
 (segment (start 142.1625 96.428) (end 143.8375 96.428) (width 0.1524) (layer "F.Cu") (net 3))
 (segment (start 144.7745 93.313) (end 145.212 93.313) (width 0.1524) (layer "F.Cu") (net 3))
 (segment (start 143.8375 96.428) (end 143.8375 94.25) (width 0.1524) (layer "F.Cu") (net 3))
 (segment (start 143.8375 94.25) (end 144.7745 93.313) (width 0.1524) (layer "F.Cu") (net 3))
 (segment (start 127.225 92.178) (end 129.865 92.178) (width 0.1524) (layer "F.Cu") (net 6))
 (segment (start 129.865 92.178) (end 130 92.043) (width 0.1524) (layer "F.Cu") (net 6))
 (segment (start 129.865 93.448) (end 130 93.313) (width 0.1524) (layer "F.Cu") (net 7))
 (segment (start 127.225 93.448) (end 129.865 93.448) (width 0.1524) (layer "F.Cu") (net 7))
 (segment (start 136 100.0875) (end 133.516966 100.0875) (width 0.1524) (layer "F.Cu") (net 9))
 (segment (start 136 100.0875) (end 136.8375 100.0875) (width 0.1524) (layer "F.Cu") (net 9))
 (segment (start 136.8375 100.0875) (end 137.75 101) (width 0.1524) (layer "F.Cu") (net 9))
 (segment (start 131.7089 96.613442) (end 133.739342 94.583) (width 0.1524) (layer "F.Cu") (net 9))
 (segment (start 133.516966 100.0875) (end 131.7089 98.279434) (width 0.1524) (layer "F.Cu") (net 9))
 (segment (start 131.7089 98.279434) (end 131.7089 96.613442) (width 0.1524) (layer "F.Cu") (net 9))
 (segment (start 133.739342 94.583) (end 134.95 94.583) (width 0.1524) (layer "F.Cu") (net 9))
 (segment (start 130.925 95.508) (end 130.925 97.5) (width 0.1524) (layer "F.Cu") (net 8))
 (segment (start 130 94.583) (end 130.925 95.508) (width 0.1524) (layer "F.Cu") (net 8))
 (segment (start 138.4262 95.91907) (end 139.01133 96.5042) (width 0.1524) (layer "F.Cu") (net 4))
 (segment (start 136.5 92.618001) (end 136.5 93.6518) (width 0.1524) (layer "F.Cu") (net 4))
 (segment (start 134.95 92.043) (end 135.924999 92.043) (width 0.1524) (layer "F.Cu") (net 4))
 (segment (start 135.924999 92.043) (end 136.5 92.618001) (width 0.1524) (layer "F.Cu") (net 4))
 (segment (start 138.157664 94.4018) (end 138.4262 94.670336) (width 0.1524) (layer "F.Cu") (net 4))
 (segment (start 139.01133 96.5042) (end 140.2613 96.5042) (width 0.1524) (layer "F.Cu") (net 4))
 (segment (start 138.4262 94.670336) (end 138.4262 95.91907) (width 0.1524) (layer "F.Cu") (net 4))
 (segment (start 136.5 93.6518) (end 137.25 94.4018) (width 0.1524) (layer "F.Cu") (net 4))
 (segment (start 140.2613 96.5042) (end 140.3375 96.428) (width 0.1524) (layer "F.Cu") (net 4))
 (segment (start 137.25 94.4018) (end 138.157664 94.4018) (width 0.1524) (layer "F.Cu") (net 4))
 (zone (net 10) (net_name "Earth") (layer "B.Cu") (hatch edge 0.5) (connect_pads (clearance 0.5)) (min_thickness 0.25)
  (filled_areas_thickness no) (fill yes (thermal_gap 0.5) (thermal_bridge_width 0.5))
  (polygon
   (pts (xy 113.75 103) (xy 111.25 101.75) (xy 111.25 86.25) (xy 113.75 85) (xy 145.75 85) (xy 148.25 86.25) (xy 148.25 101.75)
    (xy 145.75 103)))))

